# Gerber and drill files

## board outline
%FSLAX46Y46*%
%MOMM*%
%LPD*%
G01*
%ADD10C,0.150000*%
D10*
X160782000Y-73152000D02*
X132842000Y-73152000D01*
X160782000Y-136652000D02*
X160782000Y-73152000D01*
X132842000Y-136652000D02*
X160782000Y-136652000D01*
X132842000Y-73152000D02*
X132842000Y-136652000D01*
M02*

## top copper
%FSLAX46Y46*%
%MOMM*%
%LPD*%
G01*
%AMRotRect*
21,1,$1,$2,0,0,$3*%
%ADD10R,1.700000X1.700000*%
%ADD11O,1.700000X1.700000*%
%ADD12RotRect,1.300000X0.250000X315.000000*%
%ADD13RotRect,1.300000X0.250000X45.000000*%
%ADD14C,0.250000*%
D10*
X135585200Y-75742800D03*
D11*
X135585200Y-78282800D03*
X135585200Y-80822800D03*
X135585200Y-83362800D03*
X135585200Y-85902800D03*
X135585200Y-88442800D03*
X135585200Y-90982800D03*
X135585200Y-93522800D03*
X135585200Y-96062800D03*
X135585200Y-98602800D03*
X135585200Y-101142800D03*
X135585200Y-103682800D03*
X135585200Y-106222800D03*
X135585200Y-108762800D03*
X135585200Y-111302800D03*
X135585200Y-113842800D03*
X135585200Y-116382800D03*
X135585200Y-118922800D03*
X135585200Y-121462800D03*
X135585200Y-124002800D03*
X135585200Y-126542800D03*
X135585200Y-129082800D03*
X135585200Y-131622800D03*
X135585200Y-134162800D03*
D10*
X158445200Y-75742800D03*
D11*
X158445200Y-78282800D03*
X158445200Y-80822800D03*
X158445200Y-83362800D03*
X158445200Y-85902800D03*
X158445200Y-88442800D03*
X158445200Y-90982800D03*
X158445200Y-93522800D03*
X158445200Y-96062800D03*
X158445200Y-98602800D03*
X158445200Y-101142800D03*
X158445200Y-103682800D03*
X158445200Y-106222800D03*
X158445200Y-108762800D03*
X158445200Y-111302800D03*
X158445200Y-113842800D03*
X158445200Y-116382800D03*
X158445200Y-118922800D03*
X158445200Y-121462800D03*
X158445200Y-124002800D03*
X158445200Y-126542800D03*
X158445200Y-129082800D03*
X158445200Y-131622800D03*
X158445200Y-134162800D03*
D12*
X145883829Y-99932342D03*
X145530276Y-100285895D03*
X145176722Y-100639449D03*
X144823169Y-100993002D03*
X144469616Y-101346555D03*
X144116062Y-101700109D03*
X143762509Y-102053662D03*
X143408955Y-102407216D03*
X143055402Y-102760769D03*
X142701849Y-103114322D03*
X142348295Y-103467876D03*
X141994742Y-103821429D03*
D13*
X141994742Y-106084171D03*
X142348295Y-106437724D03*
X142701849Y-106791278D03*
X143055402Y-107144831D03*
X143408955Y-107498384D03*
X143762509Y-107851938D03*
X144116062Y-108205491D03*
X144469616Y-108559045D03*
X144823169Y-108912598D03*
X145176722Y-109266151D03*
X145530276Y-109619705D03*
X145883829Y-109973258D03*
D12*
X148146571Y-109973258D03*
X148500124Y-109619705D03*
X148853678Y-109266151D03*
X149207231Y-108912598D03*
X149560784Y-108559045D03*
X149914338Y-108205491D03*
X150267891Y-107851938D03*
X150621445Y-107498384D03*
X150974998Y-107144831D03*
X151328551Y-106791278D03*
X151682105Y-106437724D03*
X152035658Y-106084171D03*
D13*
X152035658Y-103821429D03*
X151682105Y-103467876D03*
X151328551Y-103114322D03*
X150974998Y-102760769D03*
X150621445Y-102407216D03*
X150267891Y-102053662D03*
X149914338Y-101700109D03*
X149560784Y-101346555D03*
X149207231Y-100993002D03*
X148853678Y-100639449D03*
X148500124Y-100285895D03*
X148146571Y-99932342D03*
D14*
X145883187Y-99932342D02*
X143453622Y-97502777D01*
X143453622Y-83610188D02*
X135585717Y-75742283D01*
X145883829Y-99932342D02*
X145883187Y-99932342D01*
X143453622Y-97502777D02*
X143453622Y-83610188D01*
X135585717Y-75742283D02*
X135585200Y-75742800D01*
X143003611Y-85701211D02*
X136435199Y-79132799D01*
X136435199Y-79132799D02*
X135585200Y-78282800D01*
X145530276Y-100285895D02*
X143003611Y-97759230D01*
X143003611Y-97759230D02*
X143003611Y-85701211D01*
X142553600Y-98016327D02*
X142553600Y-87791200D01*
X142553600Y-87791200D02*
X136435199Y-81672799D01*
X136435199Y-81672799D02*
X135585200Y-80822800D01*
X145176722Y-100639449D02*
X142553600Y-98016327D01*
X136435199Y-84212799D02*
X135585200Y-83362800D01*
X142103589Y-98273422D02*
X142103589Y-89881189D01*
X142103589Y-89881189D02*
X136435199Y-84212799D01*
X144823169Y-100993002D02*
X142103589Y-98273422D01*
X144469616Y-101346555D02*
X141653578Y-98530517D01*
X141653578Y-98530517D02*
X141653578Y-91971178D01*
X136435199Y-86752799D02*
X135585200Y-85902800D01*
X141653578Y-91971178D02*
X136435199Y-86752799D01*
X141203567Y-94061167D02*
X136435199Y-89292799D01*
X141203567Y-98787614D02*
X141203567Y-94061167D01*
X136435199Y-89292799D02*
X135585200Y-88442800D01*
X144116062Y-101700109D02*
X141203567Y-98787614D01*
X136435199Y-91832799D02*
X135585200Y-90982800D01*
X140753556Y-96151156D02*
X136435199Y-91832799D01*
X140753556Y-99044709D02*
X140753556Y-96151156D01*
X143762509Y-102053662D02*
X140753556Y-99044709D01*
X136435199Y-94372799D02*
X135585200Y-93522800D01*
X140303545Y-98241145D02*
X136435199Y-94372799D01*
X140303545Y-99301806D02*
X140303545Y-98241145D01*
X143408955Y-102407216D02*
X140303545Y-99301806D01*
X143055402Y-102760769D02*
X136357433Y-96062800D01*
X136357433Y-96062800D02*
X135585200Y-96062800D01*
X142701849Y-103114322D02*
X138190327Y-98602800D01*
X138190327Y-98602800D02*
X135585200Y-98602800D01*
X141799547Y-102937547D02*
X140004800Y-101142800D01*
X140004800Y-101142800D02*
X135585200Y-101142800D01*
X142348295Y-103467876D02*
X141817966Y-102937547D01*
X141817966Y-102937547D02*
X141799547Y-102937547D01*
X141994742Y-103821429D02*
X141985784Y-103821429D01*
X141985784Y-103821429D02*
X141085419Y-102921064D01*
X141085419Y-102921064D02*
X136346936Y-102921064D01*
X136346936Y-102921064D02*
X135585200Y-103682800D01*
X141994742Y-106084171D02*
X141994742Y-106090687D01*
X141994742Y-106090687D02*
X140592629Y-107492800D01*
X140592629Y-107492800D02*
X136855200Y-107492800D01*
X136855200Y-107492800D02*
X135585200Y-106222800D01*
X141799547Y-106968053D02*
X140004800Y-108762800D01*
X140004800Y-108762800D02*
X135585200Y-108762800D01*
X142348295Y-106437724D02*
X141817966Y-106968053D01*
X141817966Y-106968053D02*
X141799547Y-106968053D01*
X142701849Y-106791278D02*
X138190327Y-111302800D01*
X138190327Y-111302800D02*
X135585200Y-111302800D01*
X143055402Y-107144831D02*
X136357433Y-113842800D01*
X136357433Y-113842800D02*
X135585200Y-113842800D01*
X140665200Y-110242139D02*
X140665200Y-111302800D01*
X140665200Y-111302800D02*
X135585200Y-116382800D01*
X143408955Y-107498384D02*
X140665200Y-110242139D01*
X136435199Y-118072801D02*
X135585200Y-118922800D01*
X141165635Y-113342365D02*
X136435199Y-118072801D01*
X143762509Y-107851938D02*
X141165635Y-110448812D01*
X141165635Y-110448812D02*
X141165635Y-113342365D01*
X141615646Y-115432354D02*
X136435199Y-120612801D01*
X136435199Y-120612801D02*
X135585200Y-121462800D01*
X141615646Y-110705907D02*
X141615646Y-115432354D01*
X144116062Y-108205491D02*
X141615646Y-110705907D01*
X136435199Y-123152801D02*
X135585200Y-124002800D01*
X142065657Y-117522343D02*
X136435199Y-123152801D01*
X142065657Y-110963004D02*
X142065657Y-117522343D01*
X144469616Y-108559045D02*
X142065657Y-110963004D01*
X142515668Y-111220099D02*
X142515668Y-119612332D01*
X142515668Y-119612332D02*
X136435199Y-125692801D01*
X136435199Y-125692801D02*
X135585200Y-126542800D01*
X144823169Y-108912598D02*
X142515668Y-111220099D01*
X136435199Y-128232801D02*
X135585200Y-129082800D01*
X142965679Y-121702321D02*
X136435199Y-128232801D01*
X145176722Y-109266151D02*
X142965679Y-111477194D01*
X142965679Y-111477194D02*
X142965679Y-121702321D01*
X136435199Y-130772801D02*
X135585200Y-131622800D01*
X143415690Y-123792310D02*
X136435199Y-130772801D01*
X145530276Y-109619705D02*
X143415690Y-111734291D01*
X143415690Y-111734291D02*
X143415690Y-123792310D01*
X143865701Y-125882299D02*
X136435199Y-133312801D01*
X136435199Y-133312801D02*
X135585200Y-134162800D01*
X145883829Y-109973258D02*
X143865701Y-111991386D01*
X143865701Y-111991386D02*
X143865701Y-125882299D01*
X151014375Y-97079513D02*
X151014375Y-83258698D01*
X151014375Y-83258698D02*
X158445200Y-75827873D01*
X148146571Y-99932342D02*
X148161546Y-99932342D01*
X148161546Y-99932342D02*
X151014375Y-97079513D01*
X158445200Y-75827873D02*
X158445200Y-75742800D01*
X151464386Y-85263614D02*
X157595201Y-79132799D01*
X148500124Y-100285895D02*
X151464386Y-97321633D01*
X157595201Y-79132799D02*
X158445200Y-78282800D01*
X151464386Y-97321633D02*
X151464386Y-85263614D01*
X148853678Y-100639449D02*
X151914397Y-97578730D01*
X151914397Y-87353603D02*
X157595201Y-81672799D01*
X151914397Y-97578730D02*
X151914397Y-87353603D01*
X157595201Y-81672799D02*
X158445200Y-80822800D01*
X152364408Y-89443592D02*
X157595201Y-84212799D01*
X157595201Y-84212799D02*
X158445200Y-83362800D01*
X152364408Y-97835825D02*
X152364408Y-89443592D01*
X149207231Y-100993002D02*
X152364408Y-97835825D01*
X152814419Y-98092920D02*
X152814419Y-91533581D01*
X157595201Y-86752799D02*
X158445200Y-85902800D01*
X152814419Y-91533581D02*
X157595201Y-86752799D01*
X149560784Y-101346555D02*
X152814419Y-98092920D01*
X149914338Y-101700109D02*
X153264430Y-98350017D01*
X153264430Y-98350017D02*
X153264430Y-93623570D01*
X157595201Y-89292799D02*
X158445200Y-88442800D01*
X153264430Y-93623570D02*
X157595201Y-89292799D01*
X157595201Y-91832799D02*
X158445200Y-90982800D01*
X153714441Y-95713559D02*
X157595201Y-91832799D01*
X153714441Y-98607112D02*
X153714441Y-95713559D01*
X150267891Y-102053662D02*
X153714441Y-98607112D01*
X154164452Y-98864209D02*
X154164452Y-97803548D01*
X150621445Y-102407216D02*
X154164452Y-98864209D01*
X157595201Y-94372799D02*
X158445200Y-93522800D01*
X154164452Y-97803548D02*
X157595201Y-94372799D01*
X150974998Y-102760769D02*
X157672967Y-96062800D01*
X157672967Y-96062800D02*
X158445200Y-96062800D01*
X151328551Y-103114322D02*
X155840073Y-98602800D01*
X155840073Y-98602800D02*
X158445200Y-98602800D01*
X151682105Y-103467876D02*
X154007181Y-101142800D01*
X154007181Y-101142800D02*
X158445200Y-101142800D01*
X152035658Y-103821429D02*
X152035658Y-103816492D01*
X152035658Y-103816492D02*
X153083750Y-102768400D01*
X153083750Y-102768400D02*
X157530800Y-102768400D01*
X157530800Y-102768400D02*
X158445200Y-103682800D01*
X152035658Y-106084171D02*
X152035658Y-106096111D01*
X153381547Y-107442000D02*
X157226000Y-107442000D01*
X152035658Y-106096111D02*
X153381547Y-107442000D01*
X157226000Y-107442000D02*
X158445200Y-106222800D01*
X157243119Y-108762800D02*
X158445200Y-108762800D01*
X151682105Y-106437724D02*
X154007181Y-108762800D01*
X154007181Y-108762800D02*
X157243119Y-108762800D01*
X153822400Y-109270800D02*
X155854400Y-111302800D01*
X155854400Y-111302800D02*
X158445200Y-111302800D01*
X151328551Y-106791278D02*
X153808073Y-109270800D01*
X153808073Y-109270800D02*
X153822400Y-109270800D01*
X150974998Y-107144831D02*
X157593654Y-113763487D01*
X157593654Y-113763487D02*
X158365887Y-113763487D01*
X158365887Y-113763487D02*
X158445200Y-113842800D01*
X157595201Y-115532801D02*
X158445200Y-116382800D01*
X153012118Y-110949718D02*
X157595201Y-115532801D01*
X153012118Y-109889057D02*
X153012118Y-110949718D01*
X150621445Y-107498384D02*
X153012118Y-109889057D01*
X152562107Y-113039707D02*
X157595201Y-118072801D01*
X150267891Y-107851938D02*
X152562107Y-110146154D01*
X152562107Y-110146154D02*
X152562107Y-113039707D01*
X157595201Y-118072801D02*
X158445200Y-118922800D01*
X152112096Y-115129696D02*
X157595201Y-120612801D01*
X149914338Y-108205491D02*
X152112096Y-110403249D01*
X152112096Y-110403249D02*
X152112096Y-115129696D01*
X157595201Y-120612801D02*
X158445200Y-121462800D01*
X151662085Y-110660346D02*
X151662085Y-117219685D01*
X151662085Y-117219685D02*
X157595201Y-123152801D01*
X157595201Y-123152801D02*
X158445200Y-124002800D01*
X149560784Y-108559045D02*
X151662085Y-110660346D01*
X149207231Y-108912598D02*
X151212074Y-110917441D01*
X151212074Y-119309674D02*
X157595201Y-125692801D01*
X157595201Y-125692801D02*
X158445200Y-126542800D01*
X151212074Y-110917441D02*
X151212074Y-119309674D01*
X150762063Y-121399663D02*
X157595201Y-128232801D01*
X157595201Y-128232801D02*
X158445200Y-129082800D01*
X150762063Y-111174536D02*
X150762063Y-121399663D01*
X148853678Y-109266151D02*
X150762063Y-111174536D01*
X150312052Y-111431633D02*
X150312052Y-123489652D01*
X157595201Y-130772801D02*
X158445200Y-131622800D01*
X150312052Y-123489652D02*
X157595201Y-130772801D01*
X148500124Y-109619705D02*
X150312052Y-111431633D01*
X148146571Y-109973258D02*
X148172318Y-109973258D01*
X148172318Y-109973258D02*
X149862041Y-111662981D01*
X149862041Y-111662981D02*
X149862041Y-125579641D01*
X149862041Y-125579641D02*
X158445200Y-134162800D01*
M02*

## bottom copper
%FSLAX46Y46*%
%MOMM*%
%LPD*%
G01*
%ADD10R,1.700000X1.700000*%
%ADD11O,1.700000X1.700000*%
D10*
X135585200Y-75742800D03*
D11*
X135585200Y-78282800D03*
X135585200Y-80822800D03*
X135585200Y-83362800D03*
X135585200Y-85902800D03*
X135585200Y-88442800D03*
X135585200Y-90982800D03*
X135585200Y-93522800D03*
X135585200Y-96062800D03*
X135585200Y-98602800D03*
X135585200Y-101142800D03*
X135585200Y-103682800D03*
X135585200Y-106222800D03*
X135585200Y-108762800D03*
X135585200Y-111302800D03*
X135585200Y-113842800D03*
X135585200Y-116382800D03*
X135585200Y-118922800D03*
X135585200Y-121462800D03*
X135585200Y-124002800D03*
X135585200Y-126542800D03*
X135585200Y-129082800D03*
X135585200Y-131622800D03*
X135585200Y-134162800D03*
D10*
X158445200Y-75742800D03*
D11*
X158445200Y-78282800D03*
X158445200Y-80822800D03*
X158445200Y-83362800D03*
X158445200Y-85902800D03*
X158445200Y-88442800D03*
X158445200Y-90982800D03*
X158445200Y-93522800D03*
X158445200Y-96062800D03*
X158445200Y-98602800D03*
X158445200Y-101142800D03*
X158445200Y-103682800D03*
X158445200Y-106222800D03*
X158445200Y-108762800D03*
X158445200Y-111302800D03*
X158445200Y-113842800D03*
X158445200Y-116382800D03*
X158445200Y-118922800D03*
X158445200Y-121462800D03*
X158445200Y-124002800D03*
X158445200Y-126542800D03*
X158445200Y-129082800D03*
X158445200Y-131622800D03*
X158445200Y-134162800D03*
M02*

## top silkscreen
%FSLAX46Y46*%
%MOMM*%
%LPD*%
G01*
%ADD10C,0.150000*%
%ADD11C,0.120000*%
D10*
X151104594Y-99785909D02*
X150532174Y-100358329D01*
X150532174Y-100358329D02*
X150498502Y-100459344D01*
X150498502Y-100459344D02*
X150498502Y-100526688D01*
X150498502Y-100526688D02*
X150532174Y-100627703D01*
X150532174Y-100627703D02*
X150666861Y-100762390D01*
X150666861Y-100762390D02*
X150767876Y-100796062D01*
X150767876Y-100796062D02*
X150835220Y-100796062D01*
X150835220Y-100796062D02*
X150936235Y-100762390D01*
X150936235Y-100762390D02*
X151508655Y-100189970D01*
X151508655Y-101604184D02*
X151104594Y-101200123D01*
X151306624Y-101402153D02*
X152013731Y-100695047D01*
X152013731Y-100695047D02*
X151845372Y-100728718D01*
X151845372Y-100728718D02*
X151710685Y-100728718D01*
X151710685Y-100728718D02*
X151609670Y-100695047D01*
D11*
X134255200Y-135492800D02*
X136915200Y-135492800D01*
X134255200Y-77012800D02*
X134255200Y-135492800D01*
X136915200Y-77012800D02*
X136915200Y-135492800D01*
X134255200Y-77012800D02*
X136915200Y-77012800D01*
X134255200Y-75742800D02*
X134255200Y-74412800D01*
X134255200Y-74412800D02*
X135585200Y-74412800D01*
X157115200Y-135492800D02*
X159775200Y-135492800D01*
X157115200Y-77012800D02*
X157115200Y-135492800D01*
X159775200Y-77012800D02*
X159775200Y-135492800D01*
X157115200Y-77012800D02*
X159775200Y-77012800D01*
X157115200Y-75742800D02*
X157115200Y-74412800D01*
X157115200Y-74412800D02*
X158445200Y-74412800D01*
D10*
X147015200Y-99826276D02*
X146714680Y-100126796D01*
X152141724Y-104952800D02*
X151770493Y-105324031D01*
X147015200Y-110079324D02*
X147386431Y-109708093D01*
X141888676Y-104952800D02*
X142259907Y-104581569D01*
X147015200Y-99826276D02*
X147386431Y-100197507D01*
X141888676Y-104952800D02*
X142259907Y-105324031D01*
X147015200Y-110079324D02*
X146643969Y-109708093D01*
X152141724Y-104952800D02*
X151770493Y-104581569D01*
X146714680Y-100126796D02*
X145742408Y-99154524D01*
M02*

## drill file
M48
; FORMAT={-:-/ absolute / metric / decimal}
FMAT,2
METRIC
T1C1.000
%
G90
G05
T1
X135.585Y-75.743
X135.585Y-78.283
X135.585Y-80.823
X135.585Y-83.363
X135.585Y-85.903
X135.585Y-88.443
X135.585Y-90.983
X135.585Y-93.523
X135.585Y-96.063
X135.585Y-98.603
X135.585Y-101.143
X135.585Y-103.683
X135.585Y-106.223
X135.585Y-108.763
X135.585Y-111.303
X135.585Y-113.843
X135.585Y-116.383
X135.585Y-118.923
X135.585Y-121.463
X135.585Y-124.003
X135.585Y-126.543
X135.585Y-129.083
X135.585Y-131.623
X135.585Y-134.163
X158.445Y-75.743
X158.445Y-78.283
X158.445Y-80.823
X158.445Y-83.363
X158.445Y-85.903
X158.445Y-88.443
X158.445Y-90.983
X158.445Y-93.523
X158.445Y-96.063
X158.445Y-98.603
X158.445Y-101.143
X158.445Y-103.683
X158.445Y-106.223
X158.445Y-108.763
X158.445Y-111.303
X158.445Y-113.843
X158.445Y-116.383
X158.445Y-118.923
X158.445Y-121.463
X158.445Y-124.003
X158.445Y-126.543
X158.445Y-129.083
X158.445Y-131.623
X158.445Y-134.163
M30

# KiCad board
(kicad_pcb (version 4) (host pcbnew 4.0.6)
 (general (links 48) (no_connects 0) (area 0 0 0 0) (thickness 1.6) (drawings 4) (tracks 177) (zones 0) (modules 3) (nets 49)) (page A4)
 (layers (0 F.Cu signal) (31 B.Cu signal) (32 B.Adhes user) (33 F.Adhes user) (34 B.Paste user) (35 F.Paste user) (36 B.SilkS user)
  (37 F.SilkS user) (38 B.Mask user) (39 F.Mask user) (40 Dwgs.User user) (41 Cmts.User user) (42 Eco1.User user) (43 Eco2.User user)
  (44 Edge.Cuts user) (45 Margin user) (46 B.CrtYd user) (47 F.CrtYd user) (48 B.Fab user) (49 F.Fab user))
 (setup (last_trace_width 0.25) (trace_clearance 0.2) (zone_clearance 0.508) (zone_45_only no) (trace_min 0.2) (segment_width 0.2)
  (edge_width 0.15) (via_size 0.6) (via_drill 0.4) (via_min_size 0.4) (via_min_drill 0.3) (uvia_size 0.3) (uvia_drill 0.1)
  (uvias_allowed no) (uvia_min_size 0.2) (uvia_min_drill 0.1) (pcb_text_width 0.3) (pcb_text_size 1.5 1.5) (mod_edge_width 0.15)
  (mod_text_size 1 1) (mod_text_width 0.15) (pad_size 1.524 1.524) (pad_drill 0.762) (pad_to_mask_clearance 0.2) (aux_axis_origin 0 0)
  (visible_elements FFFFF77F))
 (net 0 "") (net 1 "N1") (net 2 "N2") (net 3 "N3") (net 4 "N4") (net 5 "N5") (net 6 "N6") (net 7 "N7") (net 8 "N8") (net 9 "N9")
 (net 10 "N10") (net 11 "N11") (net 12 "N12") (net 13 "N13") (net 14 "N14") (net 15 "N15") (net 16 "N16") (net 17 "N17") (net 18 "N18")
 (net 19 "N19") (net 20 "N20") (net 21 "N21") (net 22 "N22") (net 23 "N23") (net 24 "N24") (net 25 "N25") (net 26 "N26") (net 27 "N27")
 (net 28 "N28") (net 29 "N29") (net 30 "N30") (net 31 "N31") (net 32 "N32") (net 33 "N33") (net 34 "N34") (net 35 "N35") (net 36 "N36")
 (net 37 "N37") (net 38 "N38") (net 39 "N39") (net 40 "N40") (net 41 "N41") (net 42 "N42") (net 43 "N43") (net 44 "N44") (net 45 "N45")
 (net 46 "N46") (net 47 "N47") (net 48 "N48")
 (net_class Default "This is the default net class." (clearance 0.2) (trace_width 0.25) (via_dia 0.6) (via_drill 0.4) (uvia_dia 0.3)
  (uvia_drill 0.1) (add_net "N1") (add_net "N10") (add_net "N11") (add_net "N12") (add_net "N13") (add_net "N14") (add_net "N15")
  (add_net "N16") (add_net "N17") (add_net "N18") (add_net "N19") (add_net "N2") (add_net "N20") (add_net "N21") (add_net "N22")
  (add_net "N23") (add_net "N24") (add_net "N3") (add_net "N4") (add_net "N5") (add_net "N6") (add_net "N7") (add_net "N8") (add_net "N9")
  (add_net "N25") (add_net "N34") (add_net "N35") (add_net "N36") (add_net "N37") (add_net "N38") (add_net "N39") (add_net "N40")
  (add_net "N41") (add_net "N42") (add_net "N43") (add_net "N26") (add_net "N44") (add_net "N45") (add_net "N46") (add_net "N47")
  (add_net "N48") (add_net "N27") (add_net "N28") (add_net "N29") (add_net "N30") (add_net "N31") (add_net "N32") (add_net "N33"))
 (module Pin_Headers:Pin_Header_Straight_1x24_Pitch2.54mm (layer F.Cu) (at 135.5852 75.7428)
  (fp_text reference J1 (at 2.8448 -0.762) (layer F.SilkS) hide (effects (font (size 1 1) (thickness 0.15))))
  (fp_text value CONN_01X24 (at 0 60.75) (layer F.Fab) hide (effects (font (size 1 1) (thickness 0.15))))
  (fp_line (start -1.33 59.75) (end 1.33 59.75) (layer F.SilkS) (width 0.12))
  (fp_line (start -1.33 1.27) (end -1.33 59.75) (layer F.SilkS) (width 0.12))
  (fp_line (start 1.33 1.27) (end 1.33 59.75) (layer F.SilkS) (width 0.12))
  (fp_line (start -1.33 1.27) (end 1.33 1.27) (layer F.SilkS) (width 0.12))
  (fp_line (start -1.33 0) (end -1.33 -1.33) (layer F.SilkS) (width 0.12))
  (fp_line (start -1.33 -1.33) (end 0 -1.33) (layer F.SilkS) (width 0.12))
  (pad 1 thru_hole rect (at 0 0) (size 1.7 1.7) (drill 1) (layers *.Cu *.Mask) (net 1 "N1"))
  (pad 2 thru_hole oval (at 0 2.54) (size 1.7 1.7) (drill 1) (layers *.Cu *.Mask) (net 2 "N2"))
  (pad 3 thru_hole oval (at 0 5.08) (size 1.7 1.7) (drill 1) (layers *.Cu *.Mask) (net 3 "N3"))
  (pad 4 thru_hole oval (at 0 7.62) (size 1.7 1.7) (drill 1) (layers *.Cu *.Mask) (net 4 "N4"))
  (pad 5 thru_hole oval (at 0 10.16) (size 1.7 1.7) (drill 1) (layers *.Cu *.Mask) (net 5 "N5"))
  (pad 6 thru_hole oval (at 0 12.7) (size 1.7 1.7) (drill 1) (layers *.Cu *.Mask) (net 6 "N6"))
  (pad 7 thru_hole oval (at 0 15.24) (size 1.7 1.7) (drill 1) (layers *.Cu *.Mask) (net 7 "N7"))
  (pad 8 thru_hole oval (at 0 17.78) (size 1.7 1.7) (drill 1) (layers *.Cu *.Mask) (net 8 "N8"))
  (pad 9 thru_hole oval (at 0 20.32) (size 1.7 1.7) (drill 1) (layers *.Cu *.Mask) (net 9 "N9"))
  (pad 10 thru_hole oval (at 0 22.86) (size 1.7 1.7) (drill 1) (layers *.Cu *.Mask) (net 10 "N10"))
  (pad 11 thru_hole oval (at 0 25.4) (size 1.7 1.7) (drill 1) (layers *.Cu *.Mask) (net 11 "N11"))
  (pad 12 thru_hole oval (at 0 27.94) (size 1.7 1.7) (drill 1) (layers *.Cu *.Mask) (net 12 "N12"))
  (pad 13 thru_hole oval (at 0 30.48) (size 1.7 1.7) (drill 1) (layers *.Cu *.Mask) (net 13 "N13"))
  (pad 14 thru_hole oval (at 0 33.02) (size 1.7 1.7) (drill 1) (layers *.Cu *.Mask) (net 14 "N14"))
  (pad 15 thru_hole oval (at 0 35.56) (size 1.7 1.7) (drill 1) (layers *.Cu *.Mask) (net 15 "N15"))
  (pad 16 thru_hole oval (at 0 38.1) (size 1.7 1.7) (drill 1) (layers *.Cu *.Mask) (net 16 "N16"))
  (pad 17 thru_hole oval (at 0 40.64) (size 1.7 1.7) (drill 1) (layers *.Cu *.Mask) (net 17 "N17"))
  (pad 18 thru_hole oval (at 0 43.18) (size 1.7 1.7) (drill 1) (layers *.Cu *.Mask) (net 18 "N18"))
  (pad 19 thru_hole oval (at 0 45.72) (size 1.7 1.7) (drill 1) (layers *.Cu *.Mask) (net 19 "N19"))
  (pad 20 thru_hole oval (at 0 48.26) (size 1.7 1.7) (drill 1) (layers *.Cu *.Mask) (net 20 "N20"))
  (pad 21 thru_hole oval (at 0 50.8) (size 1.7 1.7) (drill 1) (layers *.Cu *.Mask) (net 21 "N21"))
  (pad 22 thru_hole oval (at 0 53.34) (size 1.7 1.7) (drill 1) (layers *.Cu *.Mask) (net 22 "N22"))
  (pad 23 thru_hole oval (at 0 55.88) (size 1.7 1.7) (drill 1) (layers *.Cu *.Mask) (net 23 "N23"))
  (pad 24 thru_hole oval (at 0 58.42) (size 1.7 1.7) (drill 1) (layers *.Cu *.Mask) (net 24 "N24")))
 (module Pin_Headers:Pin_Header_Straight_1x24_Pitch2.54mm (layer F.Cu) (at 158.4452 75.7428)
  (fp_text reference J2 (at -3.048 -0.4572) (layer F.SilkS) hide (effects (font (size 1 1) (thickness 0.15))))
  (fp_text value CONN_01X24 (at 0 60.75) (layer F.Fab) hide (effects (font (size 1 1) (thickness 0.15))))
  (fp_line (start -1.33 59.75) (end 1.33 59.75) (layer F.SilkS) (width 0.12))
  (fp_line (start -1.33 1.27) (end -1.33 59.75) (layer F.SilkS) (width 0.12))
  (fp_line (start 1.33 1.27) (end 1.33 59.75) (layer F.SilkS) (width 0.12))
  (fp_line (start -1.33 1.27) (end 1.33 1.27) (layer F.SilkS) (width 0.12))
  (fp_line (start -1.33 0) (end -1.33 -1.33) (layer F.SilkS) (width 0.12))
  (fp_line (start -1.33 -1.33) (end 0 -1.33) (layer F.SilkS) (width 0.12))
  (pad 1 thru_hole rect (at 0 0) (size 1.7 1.7) (drill 1) (layers *.Cu *.Mask) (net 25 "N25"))
  (pad 2 thru_hole oval (at 0 2.54) (size 1.7 1.7) (drill 1) (layers *.Cu *.Mask) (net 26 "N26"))
  (pad 3 thru_hole oval (at 0 5.08) (size 1.7 1.7) (drill 1) (layers *.Cu *.Mask) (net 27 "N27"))
  (pad 4 thru_hole oval (at 0 7.62) (size 1.7 1.7) (drill 1) (layers *.Cu *.Mask) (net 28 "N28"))
  (pad 5 thru_hole oval (at 0 10.16) (size 1.7 1.7) (drill 1) (layers *.Cu *.Mask) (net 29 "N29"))
  (pad 6 thru_hole oval (at 0 12.7) (size 1.7 1.7) (drill 1) (layers *.Cu *.Mask) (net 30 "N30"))
  (pad 7 thru_hole oval (at 0 15.24) (size 1.7 1.7) (drill 1) (layers *.Cu *.Mask) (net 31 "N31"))
  (pad 8 thru_hole oval (at 0 17.78) (size 1.7 1.7) (drill 1) (layers *.Cu *.Mask) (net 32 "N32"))
  (pad 9 thru_hole oval (at 0 20.32) (size 1.7 1.7) (drill 1) (layers *.Cu *.Mask) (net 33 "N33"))
  (pad 10 thru_hole oval (at 0 22.86) (size 1.7 1.7) (drill 1) (layers *.Cu *.Mask) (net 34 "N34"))
  (pad 11 thru_hole oval (at 0 25.4) (size 1.7 1.7) (drill 1) (layers *.Cu *.Mask) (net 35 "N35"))
  (pad 12 thru_hole oval (at 0 27.94) (size 1.7 1.7) (drill 1) (layers *.Cu *.Mask) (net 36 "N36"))
  (pad 13 thru_hole oval (at 0 30.48) (size 1.7 1.7) (drill 1) (layers *.Cu *.Mask) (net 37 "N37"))
  (pad 14 thru_hole oval (at 0 33.02) (size 1.7 1.7) (drill 1) (layers *.Cu *.Mask) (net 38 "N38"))
  (pad 15 thru_hole oval (at 0 35.56) (size 1.7 1.7) (drill 1) (layers *.Cu *.Mask) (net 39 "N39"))
  (pad 16 thru_hole oval (at 0 38.1) (size 1.7 1.7) (drill 1) (layers *.Cu *.Mask) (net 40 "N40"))
  (pad 17 thru_hole oval (at 0 40.64) (size 1.7 1.7) (drill 1) (layers *.Cu *.Mask) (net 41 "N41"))
  (pad 18 thru_hole oval (at 0 43.18) (size 1.7 1.7) (drill 1) (layers *.Cu *.Mask) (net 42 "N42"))
  (pad 19 thru_hole oval (at 0 45.72) (size 1.7 1.7) (drill 1) (layers *.Cu *.Mask) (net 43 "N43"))
  (pad 20 thru_hole oval (at 0 48.26) (size 1.7 1.7) (drill 1) (layers *.Cu *.Mask) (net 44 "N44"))
  (pad 21 thru_hole oval (at 0 50.8) (size 1.7 1.7) (drill 1) (layers *.Cu *.Mask) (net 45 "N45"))
  (pad 22 thru_hole oval (at 0 53.34) (size 1.7 1.7) (drill 1) (layers *.Cu *.Mask) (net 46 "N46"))
  (pad 23 thru_hole oval (at 0 55.88) (size 1.7 1.7) (drill 1) (layers *.Cu *.Mask) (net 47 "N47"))
  (pad 24 thru_hole oval (at 0 58.42) (size 1.7 1.7) (drill 1) (layers *.Cu *.Mask) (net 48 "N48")))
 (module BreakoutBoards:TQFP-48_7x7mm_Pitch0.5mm (layer F.Cu) (at 147.0152 104.9528 315)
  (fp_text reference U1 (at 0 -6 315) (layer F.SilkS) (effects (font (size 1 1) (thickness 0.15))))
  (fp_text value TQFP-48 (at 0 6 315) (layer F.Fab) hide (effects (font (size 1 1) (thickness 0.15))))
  (fp_line (start -3.625 -3.625) (end -3.625 -3.2) (layer F.SilkS) (width 0.15))
  (fp_line (start 3.625 -3.625) (end 3.625 -3.1) (layer F.SilkS) (width 0.15))
  (fp_line (start 3.625 3.625) (end 3.625 3.1) (layer F.SilkS) (width 0.15))
  (fp_line (start -3.625 3.625) (end -3.625 3.1) (layer F.SilkS) (width 0.15))
  (fp_line (start -3.625 -3.625) (end -3.1 -3.625) (layer F.SilkS) (width 0.15))
  (fp_line (start -3.625 3.625) (end -3.1 3.625) (layer F.SilkS) (width 0.15))
  (fp_line (start 3.625 3.625) (end 3.1 3.625) (layer F.SilkS) (width 0.15))
  (fp_line (start 3.625 -3.625) (end 3.1 -3.625) (layer F.SilkS) (width 0.15))
  (fp_line (start -3.625 -3.2) (end -5 -3.2) (layer F.SilkS) (width 0.15))
  (pad 1 smd rect (at -4.35 -2.75 315) (size 1.3 0.25) (layers F.Cu F.Paste F.Mask) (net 1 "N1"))
  (pad 2 smd rect (at -4.35 -2.25 315) (size 1.3 0.25) (layers F.Cu F.Paste F.Mask) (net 2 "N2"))
  (pad 3 smd rect (at -4.35 -1.75 315) (size 1.3 0.25) (layers F.Cu F.Paste F.Mask) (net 3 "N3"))
  (pad 4 smd rect (at -4.35 -1.25 315) (size 1.3 0.25) (layers F.Cu F.Paste F.Mask) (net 4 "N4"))
  (pad 5 smd rect (at -4.35 -0.75 315) (size 1.3 0.25) (layers F.Cu F.Paste F.Mask) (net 5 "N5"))
  (pad 6 smd rect (at -4.35 -0.25 315) (size 1.3 0.25) (layers F.Cu F.Paste F.Mask) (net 6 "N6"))
  (pad 7 smd rect (at -4.35 0.25 315) (size 1.3 0.25) (layers F.Cu F.Paste F.Mask) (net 7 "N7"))
  (pad 8 smd rect (at -4.35 0.75 315) (size 1.3 0.25) (layers F.Cu F.Paste F.Mask) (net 8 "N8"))
  (pad 9 smd rect (at -4.35 1.25 315) (size 1.3 0.25) (layers F.Cu F.Paste F.Mask) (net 9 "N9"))
  (pad 10 smd rect (at -4.35 1.75 315) (size 1.3 0.25) (layers F.Cu F.Paste F.Mask) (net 10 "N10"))
  (pad 11 smd rect (at -4.35 2.25 315) (size 1.3 0.25) (layers F.Cu F.Paste F.Mask) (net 11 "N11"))
  (pad 12 smd rect (at -4.35 2.75 315) (size 1.3 0.25) (layers F.Cu F.Paste F.Mask) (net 12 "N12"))
  (pad 13 smd rect (at -2.75 4.35 45) (size 1.3 0.25) (layers F.Cu F.Paste F.Mask) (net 13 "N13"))
  (pad 14 smd rect (at -2.25 4.35 45) (size 1.3 0.25) (layers F.Cu F.Paste F.Mask) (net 14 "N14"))
  (pad 15 smd rect (at -1.75 4.35 45) (size 1.3 0.25) (layers F.Cu F.Paste F.Mask) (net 15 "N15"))
  (pad 16 smd rect (at -1.25 4.35 45) (size 1.3 0.25) (layers F.Cu F.Paste F.Mask) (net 16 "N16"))
  (pad 17 smd rect (at -0.75 4.35 45) (size 1.3 0.25) (layers F.Cu F.Paste F.Mask) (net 17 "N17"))
  (pad 18 smd rect (at -0.25 4.35 45) (size 1.3 0.25) (layers F.Cu F.Paste F.Mask) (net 18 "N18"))
  (pad 19 smd rect (at 0.25 4.35 45) (size 1.3 0.25) (layers F.Cu F.Paste F.Mask) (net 19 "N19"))
  (pad 20 smd rect (at 0.75 4.35 45) (size 1.3 0.25) (layers F.Cu F.Paste F.Mask) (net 20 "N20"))
  (pad 21 smd rect (at 1.25 4.35 45) (size 1.3 0.25) (layers F.Cu F.Paste F.Mask) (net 21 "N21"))
  (pad 22 smd rect (at 1.75 4.35 45) (size 1.3 0.25) (layers F.Cu F.Paste F.Mask) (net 22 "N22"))
  (pad 23 smd rect (at 2.25 4.35 45) (size 1.3 0.25) (layers F.Cu F.Paste F.Mask) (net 23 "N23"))
  (pad 24 smd rect (at 2.75 4.35 45) (size 1.3 0.25) (layers F.Cu F.Paste F.Mask) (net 24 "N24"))
  (pad 25 smd rect (at 4.35 2.75 315) (size 1.3 0.25) (layers F.Cu F.Paste F.Mask) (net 48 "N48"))
  (pad 26 smd rect (at 4.35 2.25 315) (size 1.3 0.25) (layers F.Cu F.Paste F.Mask) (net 47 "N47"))
  (pad 27 smd rect (at 4.35 1.75 315) (size 1.3 0.25) (layers F.Cu F.Paste F.Mask) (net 46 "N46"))
  (pad 28 smd rect (at 4.35 1.25 315) (size 1.3 0.25) (layers F.Cu F.Paste F.Mask) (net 45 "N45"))
  (pad 29 smd rect (at 4.35 0.75 315) (size 1.3 0.25) (layers F.Cu F.Paste F.Mask) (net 44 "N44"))
  (pad 30 smd rect (at 4.35 0.25 315) (size 1.3 0.25) (layers F.Cu F.Paste F.Mask) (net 43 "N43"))
  (pad 31 smd rect (at 4.35 -0.25 315) (size 1.3 0.25) (layers F.Cu F.Paste F.Mask) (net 42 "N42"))
  (pad 32 smd rect (at 4.35 -0.75 315) (size 1.3 0.25) (layers F.Cu F.Paste F.Mask) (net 41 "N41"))
  (pad 33 smd rect (at 4.35 -1.25 315) (size 1.3 0.25) (layers F.Cu F.Paste F.Mask) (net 40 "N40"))
  (pad 34 smd rect (at 4.35 -1.75 315) (size 1.3 0.25) (layers F.Cu F.Paste F.Mask) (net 39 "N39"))
  (pad 35 smd rect (at 4.35 -2.25 315) (size 1.3 0.25) (layers F.Cu F.Paste F.Mask) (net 38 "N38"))
  (pad 36 smd rect (at 4.35 -2.75 315) (size 1.3 0.25) (layers F.Cu F.Paste F.Mask) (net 37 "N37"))
  (pad 37 smd rect (at 2.75 -4.35 45) (size 1.3 0.25) (layers F.Cu F.Paste F.Mask) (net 36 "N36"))
  (pad 38 smd rect (at 2.25 -4.35 45) (size 1.3 0.25) (layers F.Cu F.Paste F.Mask) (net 35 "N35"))
  (pad 39 smd rect (at 1.75 -4.35 45) (size 1.3 0.25) (layers F.Cu F.Paste F.Mask) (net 34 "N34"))
  (pad 40 smd rect (at 1.25 -4.35 45) (size 1.3 0.25) (layers F.Cu F.Paste F.Mask) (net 33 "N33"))
  (pad 41 smd rect (at 0.75 -4.35 45) (size 1.3 0.25) (layers F.Cu F.Paste F.Mask) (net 32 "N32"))
  (pad 42 smd rect (at 0.25 -4.35 45) (size 1.3 0.25) (layers F.Cu F.Paste F.Mask) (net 31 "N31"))
  (pad 43 smd rect (at -0.25 -4.35 45) (size 1.3 0.25) (layers F.Cu F.Paste F.Mask) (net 30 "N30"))
  (pad 44 smd rect (at -0.75 -4.35 45) (size 1.3 0.25) (layers F.Cu F.Paste F.Mask) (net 29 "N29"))
  (pad 45 smd rect (at -1.25 -4.35 45) (size 1.3 0.25) (layers F.Cu F.Paste F.Mask) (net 28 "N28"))
  (pad 46 smd rect (at -1.75 -4.35 45) (size 1.3 0.25) (layers F.Cu F.Paste F.Mask) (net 27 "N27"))
  (pad 47 smd rect (at -2.25 -4.35 45) (size 1.3 0.25) (layers F.Cu F.Paste F.Mask) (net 26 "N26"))
  (pad 48 smd rect (at -2.75 -4.35 45) (size 1.3 0.25) (layers F.Cu F.Paste F.Mask) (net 25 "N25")))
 (gr_line (start 160.782 73.152) (end 132.842 73.152) (angle 90) (layer Edge.Cuts) (width 0.15))
 (gr_line (start 160.782 136.652) (end 160.782 73.152) (angle 90) (layer Edge.Cuts) (width 0.15))
 (gr_line (start 132.842 136.652) (end 160.782 136.652) (angle 90) (layer Edge.Cuts) (width 0.15))
 (gr_line (start 132.842 73.152) (end 132.842 136.652) (angle 90) (layer Edge.Cuts) (width 0.15))
 (segment (start 145.883187 99.932342) (end 143.453622 97.502777) (width 0.25) (layer F.Cu) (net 1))
 (segment (start 143.453622 83.610188) (end 135.585717 75.742283) (width 0.25) (layer F.Cu) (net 1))
 (segment (start 145.883829 99.932342) (end 145.883187 99.932342) (width 0.25) (layer F.Cu) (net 1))
 (segment (start 143.453622 97.502777) (end 143.453622 83.610188) (width 0.25) (layer F.Cu) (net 1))
 (segment (start 135.585717 75.742283) (end 135.5852 75.7428) (width 0.25) (layer F.Cu) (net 1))
 (segment (start 143.003611 85.701211) (end 136.435199 79.132799) (width 0.25) (layer F.Cu) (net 2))
 (segment (start 136.435199 79.132799) (end 135.5852 78.2828) (width 0.25) (layer F.Cu) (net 2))
 (segment (start 145.530276 100.285895) (end 143.003611 97.75923) (width 0.25) (layer F.Cu) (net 2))
 (segment (start 143.003611 97.75923) (end 143.003611 85.701211) (width 0.25) (layer F.Cu) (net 2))
 (segment (start 142.5536 98.016327) (end 142.5536 87.7912) (width 0.25) (layer F.Cu) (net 3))
 (segment (start 142.5536 87.7912) (end 136.435199 81.672799) (width 0.25) (layer F.Cu) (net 3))
 (segment (start 136.435199 81.672799) (end 135.5852 80.8228) (width 0.25) (layer F.Cu) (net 3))
 (segment (start 145.176722 100.639449) (end 142.5536 98.016327) (width 0.25) (layer F.Cu) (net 3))
 (segment (start 136.435199 84.212799) (end 135.5852 83.3628) (width 0.25) (layer F.Cu) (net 4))
 (segment (start 142.103589 98.273422) (end 142.103589 89.881189) (width 0.25) (layer F.Cu) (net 4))
 (segment (start 142.103589 89.881189) (end 136.435199 84.212799) (width 0.25) (layer F.Cu) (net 4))
 (segment (start 144.823169 100.993002) (end 142.103589 98.273422) (width 0.25) (layer F.Cu) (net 4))
 (segment (start 144.469616 101.346555) (end 141.653578 98.530517) (width 0.25) (layer F.Cu) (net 5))
 (segment (start 141.653578 98.530517) (end 141.653578 91.971178) (width 0.25) (layer F.Cu) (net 5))
 (segment (start 136.435199 86.752799) (end 135.5852 85.9028) (width 0.25) (layer F.Cu) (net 5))
 (segment (start 141.653578 91.971178) (end 136.435199 86.752799) (width 0.25) (layer F.Cu) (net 5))
 (segment (start 141.203567 94.061167) (end 136.435199 89.292799) (width 0.25) (layer F.Cu) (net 6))
 (segment (start 141.203567 98.787614) (end 141.203567 94.061167) (width 0.25) (layer F.Cu) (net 6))
 (segment (start 136.435199 89.292799) (end 135.5852 88.4428) (width 0.25) (layer F.Cu) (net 6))
 (segment (start 144.116062 101.700109) (end 141.203567 98.787614) (width 0.25) (layer F.Cu) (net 6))
 (segment (start 136.435199 91.832799) (end 135.5852 90.9828) (width 0.25) (layer F.Cu) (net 7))
 (segment (start 140.753556 96.151156) (end 136.435199 91.832799) (width 0.25) (layer F.Cu) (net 7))
 (segment (start 140.753556 99.044709) (end 140.753556 96.151156) (width 0.25) (layer F.Cu) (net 7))
 (segment (start 143.762509 102.053662) (end 140.753556 99.044709) (width 0.25) (layer F.Cu) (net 7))
 (segment (start 136.435199 94.372799) (end 135.5852 93.5228) (width 0.25) (layer F.Cu) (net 8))
 (segment (start 140.303545 98.241145) (end 136.435199 94.372799) (width 0.25) (layer F.Cu) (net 8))
 (segment (start 140.303545 99.301806) (end 140.303545 98.241145) (width 0.25) (layer F.Cu) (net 8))
 (segment (start 143.408955 102.407216) (end 140.303545 99.301806) (width 0.25) (layer F.Cu) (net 8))
 (segment (start 143.055402 102.760769) (end 136.357433 96.0628) (width 0.25) (layer F.Cu) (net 9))
 (segment (start 136.357433 96.0628) (end 135.5852 96.0628) (width 0.25) (layer F.Cu) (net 9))
 (segment (start 142.701849 103.114322) (end 138.190327 98.6028) (width 0.25) (layer F.Cu) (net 10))
 (segment (start 138.190327 98.6028) (end 135.5852 98.6028) (width 0.25) (layer F.Cu) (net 10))
 (segment (start 141.799547 102.937547) (end 140.0048 101.1428) (width 0.25) (layer F.Cu) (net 11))
 (segment (start 140.0048 101.1428) (end 135.5852 101.1428) (width 0.25) (layer F.Cu) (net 11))
 (segment (start 142.348295 103.467876) (end 141.817966 102.937547) (width 0.25) (layer F.Cu) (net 11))
 (segment (start 141.817966 102.937547) (end 141.799547 102.937547) (width 0.25) (layer F.Cu) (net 11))
 (segment (start 141.994742 103.821429) (end 141.985784 103.821429) (width 0.25) (layer F.Cu) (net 12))
 (segment (start 141.985784 103.821429) (end 141.085419 102.921064) (width 0.25) (layer F.Cu) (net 12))
 (segment (start 141.085419 102.921064) (end 136.346936 102.921064) (width 0.25) (layer F.Cu) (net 12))
 (segment (start 136.346936 102.921064) (end 135.5852 103.6828) (width 0.25) (layer F.Cu) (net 12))
 (segment (start 141.994742 106.084171) (end 141.994742 106.090687) (width 0.25) (layer F.Cu) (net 13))
 (segment (start 141.994742 106.090687) (end 140.592629 107.4928) (width 0.25) (layer F.Cu) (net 13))
 (segment (start 140.592629 107.4928) (end 136.8552 107.4928) (width 0.25) (layer F.Cu) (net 13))
 (segment (start 136.8552 107.4928) (end 135.5852 106.2228) (width 0.25) (layer F.Cu) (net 13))
 (segment (start 141.799547 106.968053) (end 140.0048 108.7628) (width 0.25) (layer F.Cu) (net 14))
 (segment (start 140.0048 108.7628) (end 135.5852 108.7628) (width 0.25) (layer F.Cu) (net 14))
 (segment (start 142.348295 106.437724) (end 141.817966 106.968053) (width 0.25) (layer F.Cu) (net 14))
 (segment (start 141.817966 106.968053) (end 141.799547 106.968053) (width 0.25) (layer F.Cu) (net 14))
 (segment (start 142.701849 106.791278) (end 138.190327 111.3028) (width 0.25) (layer F.Cu) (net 15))
 (segment (start 138.190327 111.3028) (end 135.5852 111.3028) (width 0.25) (layer F.Cu) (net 15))
 (segment (start 143.055402 107.144831) (end 136.357433 113.8428) (width 0.25) (layer F.Cu) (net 16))
 (segment (start 136.357433 113.8428) (end 135.5852 113.8428) (width 0.25) (layer F.Cu) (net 16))
 (segment (start 140.6652 110.242139) (end 140.6652 111.3028) (width 0.25) (layer F.Cu) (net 17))
 (segment (start 140.6652 111.3028) (end 135.5852 116.3828) (width 0.25) (layer F.Cu) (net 17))
 (segment (start 143.408955 107.498384) (end 140.6652 110.242139) (width 0.25) (layer F.Cu) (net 17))
 (segment (start 136.435199 118.072801) (end 135.5852 118.9228) (width 0.25) (layer F.Cu) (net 18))
 (segment (start 141.165635 113.342365) (end 136.435199 118.072801) (width 0.25) (layer F.Cu) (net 18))
 (segment (start 143.762509 107.851938) (end 141.165635 110.448812) (width 0.25) (layer F.Cu) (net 18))
 (segment (start 141.165635 110.448812) (end 141.165635 113.342365) (width 0.25) (layer F.Cu) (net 18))
 (segment (start 141.615646 115.432354) (end 136.435199 120.612801) (width 0.25) (layer F.Cu) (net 19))
 (segment (start 136.435199 120.612801) (end 135.5852 121.4628) (width 0.25) (layer F.Cu) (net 19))
 (segment (start 141.615646 110.705907) (end 141.615646 115.432354) (width 0.25) (layer F.Cu) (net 19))
 (segment (start 144.116062 108.205491) (end 141.615646 110.705907) (width 0.25) (layer F.Cu) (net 19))
 (segment (start 136.435199 123.152801) (end 135.5852 124.0028) (width 0.25) (layer F.Cu) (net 20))
 (segment (start 142.065657 117.522343) (end 136.435199 123.152801) (width 0.25) (layer F.Cu) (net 20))
 (segment (start 142.065657 110.963004) (end 142.065657 117.522343) (width 0.25) (layer F.Cu) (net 20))
 (segment (start 144.469616 108.559045) (end 142.065657 110.963004) (width 0.25) (layer F.Cu) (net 20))
 (segment (start 142.515668 111.220099) (end 142.515668 119.612332) (width 0.25) (layer F.Cu) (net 21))
 (segment (start 142.515668 119.612332) (end 136.435199 125.692801) (width 0.25) (layer F.Cu) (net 21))
 (segment (start 136.435199 125.692801) (end 135.5852 126.5428) (width 0.25) (layer F.Cu) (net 21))
 (segment (start 144.823169 108.912598) (end 142.515668 111.220099) (width 0.25) (layer F.Cu) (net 21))
 (segment (start 136.435199 128.232801) (end 135.5852 129.0828) (width 0.25) (layer F.Cu) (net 22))
 (segment (start 142.965679 121.702321) (end 136.435199 128.232801) (width 0.25) (layer F.Cu) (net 22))
 (segment (start 145.176722 109.266151) (end 142.965679 111.477194) (width 0.25) (layer F.Cu) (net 22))
 (segment (start 142.965679 111.477194) (end 142.965679 121.702321) (width 0.25) (layer F.Cu) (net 22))
 (segment (start 136.435199 130.772801) (end 135.5852 131.6228) (width 0.25) (layer F.Cu) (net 23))
 (segment (start 143.41569 123.79231) (end 136.435199 130.772801) (width 0.25) (layer F.Cu) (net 23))
 (segment (start 145.530276 109.619705) (end 143.41569 111.734291) (width 0.25) (layer F.Cu) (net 23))
 (segment (start 143.41569 111.734291) (end 143.41569 123.79231) (width 0.25) (layer F.Cu) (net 23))
 (segment (start 143.865701 125.882299) (end 136.435199 133.312801) (width 0.25) (layer F.Cu) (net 24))
 (segment (start 136.435199 133.312801) (end 135.5852 134.1628) (width 0.25) (layer F.Cu) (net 24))
 (segment (start 145.883829 109.973258) (end 143.865701 111.991386) (width 0.25) (layer F.Cu) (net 24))
 (segment (start 143.865701 111.991386) (end 143.865701 125.882299) (width 0.25) (layer F.Cu) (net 24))
 (segment (start 151.014375 97.079513) (end 151.014375 83.258698) (width 0.25) (layer F.Cu) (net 25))
 (segment (start 151.014375 83.258698) (end 158.4452 75.827873) (width 0.25) (layer F.Cu) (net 25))
 (segment (start 148.146571 99.932342) (end 148.161546 99.932342) (width 0.25) (layer F.Cu) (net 25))
 (segment (start 148.161546 99.932342) (end 151.014375 97.079513) (width 0.25) (layer F.Cu) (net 25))
 (segment (start 158.4452 75.827873) (end 158.4452 75.7428) (width 0.25) (layer F.Cu) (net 25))
 (segment (start 151.464386 85.263614) (end 157.595201 79.132799) (width 0.25) (layer F.Cu) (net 26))
 (segment (start 148.500124 100.285895) (end 151.464386 97.321633) (width 0.25) (layer F.Cu) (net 26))
 (segment (start 157.595201 79.132799) (end 158.4452 78.2828) (width 0.25) (layer F.Cu) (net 26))
 (segment (start 151.464386 97.321633) (end 151.464386 85.263614) (width 0.25) (layer F.Cu) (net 26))
 (segment (start 148.853678 100.639449) (end 151.914397 97.57873) (width 0.25) (layer F.Cu) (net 27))
 (segment (start 151.914397 87.353603) (end 157.595201 81.672799) (width 0.25) (layer F.Cu) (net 27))
 (segment (start 151.914397 97.57873) (end 151.914397 87.353603) (width 0.25) (layer F.Cu) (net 27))
 (segment (start 157.595201 81.672799) (end 158.4452 80.8228) (width 0.25) (layer F.Cu) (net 27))
 (segment (start 152.364408 89.443592) (end 157.595201 84.212799) (width 0.25) (layer F.Cu) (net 28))
 (segment (start 157.595201 84.212799) (end 158.4452 83.3628) (width 0.25) (layer F.Cu) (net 28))
 (segment (start 152.364408 97.835825) (end 152.364408 89.443592) (width 0.25) (layer F.Cu) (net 28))
 (segment (start 149.207231 100.993002) (end 152.364408 97.835825) (width 0.25) (layer F.Cu) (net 28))
 (segment (start 152.814419 98.09292) (end 152.814419 91.533581) (width 0.25) (layer F.Cu) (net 29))
 (segment (start 157.595201 86.752799) (end 158.4452 85.9028) (width 0.25) (layer F.Cu) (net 29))
 (segment (start 152.814419 91.533581) (end 157.595201 86.752799) (width 0.25) (layer F.Cu) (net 29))
 (segment (start 149.560784 101.346555) (end 152.814419 98.09292) (width 0.25) (layer F.Cu) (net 29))
 (segment (start 149.914338 101.700109) (end 153.26443 98.350017) (width 0.25) (layer F.Cu) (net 30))
 (segment (start 153.26443 98.350017) (end 153.26443 93.62357) (width 0.25) (layer F.Cu) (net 30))
 (segment (start 157.595201 89.292799) (end 158.4452 88.4428) (width 0.25) (layer F.Cu) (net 30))
 (segment (start 153.26443 93.62357) (end 157.595201 89.292799) (width 0.25) (layer F.Cu) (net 30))
 (segment (start 157.595201 91.832799) (end 158.4452 90.9828) (width 0.25) (layer F.Cu) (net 31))
 (segment (start 153.714441 95.713559) (end 157.595201 91.832799) (width 0.25) (layer F.Cu) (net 31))
 (segment (start 153.714441 98.607112) (end 153.714441 95.713559) (width 0.25) (layer F.Cu) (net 31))
 (segment (start 150.267891 102.053662) (end 153.714441 98.607112) (width 0.25) (layer F.Cu) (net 31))
 (segment (start 154.164452 98.864209) (end 154.164452 97.803548) (width 0.25) (layer F.Cu) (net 32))
 (segment (start 150.621445 102.407216) (end 154.164452 98.864209) (width 0.25) (layer F.Cu) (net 32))
 (segment (start 157.595201 94.372799) (end 158.4452 93.5228) (width 0.25) (layer F.Cu) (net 32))
 (segment (start 154.164452 97.803548) (end 157.595201 94.372799) (width 0.25) (layer F.Cu) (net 32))
 (segment (start 150.974998 102.760769) (end 157.672967 96.0628) (width 0.25) (layer F.Cu) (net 33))
 (segment (start 157.672967 96.0628) (end 158.4452 96.0628) (width 0.25) (layer F.Cu) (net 33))
 (segment (start 151.328551 103.114322) (end 155.840073 98.6028) (width 0.25) (layer F.Cu) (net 34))
 (segment (start 155.840073 98.6028) (end 158.4452 98.6028) (width 0.25) (layer F.Cu) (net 34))
 (segment (start 151.682105 103.467876) (end 154.007181 101.1428) (width 0.25) (layer F.Cu) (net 35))
 (segment (start 154.007181 101.1428) (end 158.4452 101.1428) (width 0.25) (layer F.Cu) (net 35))
 (segment (start 152.035658 103.821429) (end 152.035658 103.816492) (width 0.25) (layer F.Cu) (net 36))
 (segment (start 152.035658 103.816492) (end 153.08375 102.7684) (width 0.25) (layer F.Cu) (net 36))
 (segment (start 153.08375 102.7684) (end 157.5308 102.7684) (width 0.25) (layer F.Cu) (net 36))
 (segment (start 157.5308 102.7684) (end 158.4452 103.6828) (width 0.25) (layer F.Cu) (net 36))
 (segment (start 152.035658 106.084171) (end 152.035658 106.096111) (width 0.25) (layer F.Cu) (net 37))
 (segment (start 153.381547 107.442) (end 157.226 107.442) (width 0.25) (layer F.Cu) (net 37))
 (segment (start 152.035658 106.096111) (end 153.381547 107.442) (width 0.25) (layer F.Cu) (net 37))
 (segment (start 157.226 107.442) (end 158.4452 106.2228) (width 0.25) (layer F.Cu) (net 37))
 (segment (start 157.243119 108.7628) (end 158.4452 108.7628) (width 0.25) (layer F.Cu) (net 38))
 (segment (start 151.682105 106.437724) (end 154.007181 108.7628) (width 0.25) (layer F.Cu) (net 38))
 (segment (start 154.007181 108.7628) (end 157.243119 108.7628) (width 0.25) (layer F.Cu) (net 38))
 (segment (start 153.8224 109.2708) (end 155.8544 111.3028) (width 0.25) (layer F.Cu) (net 39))
 (segment (start 155.8544 111.3028) (end 158.4452 111.3028) (width 0.25) (layer F.Cu) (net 39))
 (segment (start 151.328551 106.791278) (end 153.808073 109.2708) (width 0.25) (layer F.Cu) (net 39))
 (segment (start 153.808073 109.2708) (end 153.8224 109.2708) (width 0.25) (layer F.Cu) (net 39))
 (segment (start 150.974998 107.144831) (end 157.593654 113.763487) (width 0.25) (layer F.Cu) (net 40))
 (segment (start 157.593654 113.763487) (end 158.365887 113.763487) (width 0.25) (layer F.Cu) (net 40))
 (segment (start 158.365887 113.763487) (end 158.4452 113.8428) (width 0.25) (layer F.Cu) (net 40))
 (segment (start 157.595201 115.532801) (end 158.4452 116.3828) (width 0.25) (layer F.Cu) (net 41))
 (segment (start 153.012118 110.949718) (end 157.595201 115.532801) (width 0.25) (layer F.Cu) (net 41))
 (segment (start 153.012118 109.889057) (end 153.012118 110.949718) (width 0.25) (layer F.Cu) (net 41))
 (segment (start 150.621445 107.498384) (end 153.012118 109.889057) (width 0.25) (layer F.Cu) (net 41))
 (segment (start 152.562107 113.039707) (end 157.595201 118.072801) (width 0.25) (layer F.Cu) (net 42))
 (segment (start 150.267891 107.851938) (end 152.562107 110.146154) (width 0.25) (layer F.Cu) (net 42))
 (segment (start 152.562107 110.146154) (end 152.562107 113.039707) (width 0.25) (layer F.Cu) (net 42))
 (segment (start 157.595201 118.072801) (end 158.4452 118.9228) (width 0.25) (layer F.Cu) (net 42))
 (segment (start 152.112096 115.129696) (end 157.595201 120.612801) (width 0.25) (layer F.Cu) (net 43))
 (segment (start 149.914338 108.205491) (end 152.112096 110.403249) (width 0.25) (layer F.Cu) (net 43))
 (segment (start 152.112096 110.403249) (end 152.112096 115.129696) (width 0.25) (layer F.Cu) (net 43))
 (segment (start 157.595201 120.612801) (end 158.4452 121.4628) (width 0.25) (layer F.Cu) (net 43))
 (segment (start 151.662085 110.660346) (end 151.662085 117.219685) (width 0.25) (layer F.Cu) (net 44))
 (segment (start 151.662085 117.219685) (end 157.595201 123.152801) (width 0.25) (layer F.Cu) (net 44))
 (segment (start 157.595201 123.152801) (end 158.4452 124.0028) (width 0.25) (layer F.Cu) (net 44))
 (segment (start 149.560784 108.559045) (end 151.662085 110.660346) (width 0.25) (layer F.Cu) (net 44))
 (segment (start 149.207231 108.912598) (end 151.212074 110.917441) (width 0.25) (layer F.Cu) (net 45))
 (segment (start 151.212074 119.309674) (end 157.595201 125.692801) (width 0.25) (layer F.Cu) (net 45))
 (segment (start 157.595201 125.692801) (end 158.4452 126.5428) (width 0.25) (layer F.Cu) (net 45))
 (segment (start 151.212074 110.917441) (end 151.212074 119.309674) (width 0.25) (layer F.Cu) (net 45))
 (segment (start 150.762063 121.399663) (end 157.595201 128.232801) (width 0.25) (layer F.Cu) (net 46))
 (segment (start 157.595201 128.232801) (end 158.4452 129.0828) (width 0.25) (layer F.Cu) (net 46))
 (segment (start 150.762063 111.174536) (end 150.762063 121.399663) (width 0.25) (layer F.Cu) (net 46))
 (segment (start 148.853678 109.266151) (end 150.762063 111.174536) (width 0.25) (layer F.Cu) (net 46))
 (segment (start 150.312052 111.431633) (end 150.312052 123.489652) (width 0.25) (layer F.Cu) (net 47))
 (segment (start 157.595201 130.772801) (end 158.4452 131.6228) (width 0.25) (layer F.Cu) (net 47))
 (segment (start 150.312052 123.489652) (end 157.595201 130.772801) (width 0.25) (layer F.Cu) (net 47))
 (segment (start 148.500124 109.619705) (end 150.312052 111.431633) (width 0.25) (layer F.Cu) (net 47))
 (segment (start 148.146571 109.973258) (end 148.172318 109.973258) (width 0.25) (layer F.Cu) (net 48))
 (segment (start 148.172318 109.973258) (end 149.862041 111.662981) (width 0.25) (layer F.Cu) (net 48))
 (segment (start 149.862041 111.662981) (end 149.862041 125.579641) (width 0.25) (layer F.Cu) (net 48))
 (segment (start 149.862041 125.579641) (end 158.4452 134.1628) (width 0.25) (layer F.Cu) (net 48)))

